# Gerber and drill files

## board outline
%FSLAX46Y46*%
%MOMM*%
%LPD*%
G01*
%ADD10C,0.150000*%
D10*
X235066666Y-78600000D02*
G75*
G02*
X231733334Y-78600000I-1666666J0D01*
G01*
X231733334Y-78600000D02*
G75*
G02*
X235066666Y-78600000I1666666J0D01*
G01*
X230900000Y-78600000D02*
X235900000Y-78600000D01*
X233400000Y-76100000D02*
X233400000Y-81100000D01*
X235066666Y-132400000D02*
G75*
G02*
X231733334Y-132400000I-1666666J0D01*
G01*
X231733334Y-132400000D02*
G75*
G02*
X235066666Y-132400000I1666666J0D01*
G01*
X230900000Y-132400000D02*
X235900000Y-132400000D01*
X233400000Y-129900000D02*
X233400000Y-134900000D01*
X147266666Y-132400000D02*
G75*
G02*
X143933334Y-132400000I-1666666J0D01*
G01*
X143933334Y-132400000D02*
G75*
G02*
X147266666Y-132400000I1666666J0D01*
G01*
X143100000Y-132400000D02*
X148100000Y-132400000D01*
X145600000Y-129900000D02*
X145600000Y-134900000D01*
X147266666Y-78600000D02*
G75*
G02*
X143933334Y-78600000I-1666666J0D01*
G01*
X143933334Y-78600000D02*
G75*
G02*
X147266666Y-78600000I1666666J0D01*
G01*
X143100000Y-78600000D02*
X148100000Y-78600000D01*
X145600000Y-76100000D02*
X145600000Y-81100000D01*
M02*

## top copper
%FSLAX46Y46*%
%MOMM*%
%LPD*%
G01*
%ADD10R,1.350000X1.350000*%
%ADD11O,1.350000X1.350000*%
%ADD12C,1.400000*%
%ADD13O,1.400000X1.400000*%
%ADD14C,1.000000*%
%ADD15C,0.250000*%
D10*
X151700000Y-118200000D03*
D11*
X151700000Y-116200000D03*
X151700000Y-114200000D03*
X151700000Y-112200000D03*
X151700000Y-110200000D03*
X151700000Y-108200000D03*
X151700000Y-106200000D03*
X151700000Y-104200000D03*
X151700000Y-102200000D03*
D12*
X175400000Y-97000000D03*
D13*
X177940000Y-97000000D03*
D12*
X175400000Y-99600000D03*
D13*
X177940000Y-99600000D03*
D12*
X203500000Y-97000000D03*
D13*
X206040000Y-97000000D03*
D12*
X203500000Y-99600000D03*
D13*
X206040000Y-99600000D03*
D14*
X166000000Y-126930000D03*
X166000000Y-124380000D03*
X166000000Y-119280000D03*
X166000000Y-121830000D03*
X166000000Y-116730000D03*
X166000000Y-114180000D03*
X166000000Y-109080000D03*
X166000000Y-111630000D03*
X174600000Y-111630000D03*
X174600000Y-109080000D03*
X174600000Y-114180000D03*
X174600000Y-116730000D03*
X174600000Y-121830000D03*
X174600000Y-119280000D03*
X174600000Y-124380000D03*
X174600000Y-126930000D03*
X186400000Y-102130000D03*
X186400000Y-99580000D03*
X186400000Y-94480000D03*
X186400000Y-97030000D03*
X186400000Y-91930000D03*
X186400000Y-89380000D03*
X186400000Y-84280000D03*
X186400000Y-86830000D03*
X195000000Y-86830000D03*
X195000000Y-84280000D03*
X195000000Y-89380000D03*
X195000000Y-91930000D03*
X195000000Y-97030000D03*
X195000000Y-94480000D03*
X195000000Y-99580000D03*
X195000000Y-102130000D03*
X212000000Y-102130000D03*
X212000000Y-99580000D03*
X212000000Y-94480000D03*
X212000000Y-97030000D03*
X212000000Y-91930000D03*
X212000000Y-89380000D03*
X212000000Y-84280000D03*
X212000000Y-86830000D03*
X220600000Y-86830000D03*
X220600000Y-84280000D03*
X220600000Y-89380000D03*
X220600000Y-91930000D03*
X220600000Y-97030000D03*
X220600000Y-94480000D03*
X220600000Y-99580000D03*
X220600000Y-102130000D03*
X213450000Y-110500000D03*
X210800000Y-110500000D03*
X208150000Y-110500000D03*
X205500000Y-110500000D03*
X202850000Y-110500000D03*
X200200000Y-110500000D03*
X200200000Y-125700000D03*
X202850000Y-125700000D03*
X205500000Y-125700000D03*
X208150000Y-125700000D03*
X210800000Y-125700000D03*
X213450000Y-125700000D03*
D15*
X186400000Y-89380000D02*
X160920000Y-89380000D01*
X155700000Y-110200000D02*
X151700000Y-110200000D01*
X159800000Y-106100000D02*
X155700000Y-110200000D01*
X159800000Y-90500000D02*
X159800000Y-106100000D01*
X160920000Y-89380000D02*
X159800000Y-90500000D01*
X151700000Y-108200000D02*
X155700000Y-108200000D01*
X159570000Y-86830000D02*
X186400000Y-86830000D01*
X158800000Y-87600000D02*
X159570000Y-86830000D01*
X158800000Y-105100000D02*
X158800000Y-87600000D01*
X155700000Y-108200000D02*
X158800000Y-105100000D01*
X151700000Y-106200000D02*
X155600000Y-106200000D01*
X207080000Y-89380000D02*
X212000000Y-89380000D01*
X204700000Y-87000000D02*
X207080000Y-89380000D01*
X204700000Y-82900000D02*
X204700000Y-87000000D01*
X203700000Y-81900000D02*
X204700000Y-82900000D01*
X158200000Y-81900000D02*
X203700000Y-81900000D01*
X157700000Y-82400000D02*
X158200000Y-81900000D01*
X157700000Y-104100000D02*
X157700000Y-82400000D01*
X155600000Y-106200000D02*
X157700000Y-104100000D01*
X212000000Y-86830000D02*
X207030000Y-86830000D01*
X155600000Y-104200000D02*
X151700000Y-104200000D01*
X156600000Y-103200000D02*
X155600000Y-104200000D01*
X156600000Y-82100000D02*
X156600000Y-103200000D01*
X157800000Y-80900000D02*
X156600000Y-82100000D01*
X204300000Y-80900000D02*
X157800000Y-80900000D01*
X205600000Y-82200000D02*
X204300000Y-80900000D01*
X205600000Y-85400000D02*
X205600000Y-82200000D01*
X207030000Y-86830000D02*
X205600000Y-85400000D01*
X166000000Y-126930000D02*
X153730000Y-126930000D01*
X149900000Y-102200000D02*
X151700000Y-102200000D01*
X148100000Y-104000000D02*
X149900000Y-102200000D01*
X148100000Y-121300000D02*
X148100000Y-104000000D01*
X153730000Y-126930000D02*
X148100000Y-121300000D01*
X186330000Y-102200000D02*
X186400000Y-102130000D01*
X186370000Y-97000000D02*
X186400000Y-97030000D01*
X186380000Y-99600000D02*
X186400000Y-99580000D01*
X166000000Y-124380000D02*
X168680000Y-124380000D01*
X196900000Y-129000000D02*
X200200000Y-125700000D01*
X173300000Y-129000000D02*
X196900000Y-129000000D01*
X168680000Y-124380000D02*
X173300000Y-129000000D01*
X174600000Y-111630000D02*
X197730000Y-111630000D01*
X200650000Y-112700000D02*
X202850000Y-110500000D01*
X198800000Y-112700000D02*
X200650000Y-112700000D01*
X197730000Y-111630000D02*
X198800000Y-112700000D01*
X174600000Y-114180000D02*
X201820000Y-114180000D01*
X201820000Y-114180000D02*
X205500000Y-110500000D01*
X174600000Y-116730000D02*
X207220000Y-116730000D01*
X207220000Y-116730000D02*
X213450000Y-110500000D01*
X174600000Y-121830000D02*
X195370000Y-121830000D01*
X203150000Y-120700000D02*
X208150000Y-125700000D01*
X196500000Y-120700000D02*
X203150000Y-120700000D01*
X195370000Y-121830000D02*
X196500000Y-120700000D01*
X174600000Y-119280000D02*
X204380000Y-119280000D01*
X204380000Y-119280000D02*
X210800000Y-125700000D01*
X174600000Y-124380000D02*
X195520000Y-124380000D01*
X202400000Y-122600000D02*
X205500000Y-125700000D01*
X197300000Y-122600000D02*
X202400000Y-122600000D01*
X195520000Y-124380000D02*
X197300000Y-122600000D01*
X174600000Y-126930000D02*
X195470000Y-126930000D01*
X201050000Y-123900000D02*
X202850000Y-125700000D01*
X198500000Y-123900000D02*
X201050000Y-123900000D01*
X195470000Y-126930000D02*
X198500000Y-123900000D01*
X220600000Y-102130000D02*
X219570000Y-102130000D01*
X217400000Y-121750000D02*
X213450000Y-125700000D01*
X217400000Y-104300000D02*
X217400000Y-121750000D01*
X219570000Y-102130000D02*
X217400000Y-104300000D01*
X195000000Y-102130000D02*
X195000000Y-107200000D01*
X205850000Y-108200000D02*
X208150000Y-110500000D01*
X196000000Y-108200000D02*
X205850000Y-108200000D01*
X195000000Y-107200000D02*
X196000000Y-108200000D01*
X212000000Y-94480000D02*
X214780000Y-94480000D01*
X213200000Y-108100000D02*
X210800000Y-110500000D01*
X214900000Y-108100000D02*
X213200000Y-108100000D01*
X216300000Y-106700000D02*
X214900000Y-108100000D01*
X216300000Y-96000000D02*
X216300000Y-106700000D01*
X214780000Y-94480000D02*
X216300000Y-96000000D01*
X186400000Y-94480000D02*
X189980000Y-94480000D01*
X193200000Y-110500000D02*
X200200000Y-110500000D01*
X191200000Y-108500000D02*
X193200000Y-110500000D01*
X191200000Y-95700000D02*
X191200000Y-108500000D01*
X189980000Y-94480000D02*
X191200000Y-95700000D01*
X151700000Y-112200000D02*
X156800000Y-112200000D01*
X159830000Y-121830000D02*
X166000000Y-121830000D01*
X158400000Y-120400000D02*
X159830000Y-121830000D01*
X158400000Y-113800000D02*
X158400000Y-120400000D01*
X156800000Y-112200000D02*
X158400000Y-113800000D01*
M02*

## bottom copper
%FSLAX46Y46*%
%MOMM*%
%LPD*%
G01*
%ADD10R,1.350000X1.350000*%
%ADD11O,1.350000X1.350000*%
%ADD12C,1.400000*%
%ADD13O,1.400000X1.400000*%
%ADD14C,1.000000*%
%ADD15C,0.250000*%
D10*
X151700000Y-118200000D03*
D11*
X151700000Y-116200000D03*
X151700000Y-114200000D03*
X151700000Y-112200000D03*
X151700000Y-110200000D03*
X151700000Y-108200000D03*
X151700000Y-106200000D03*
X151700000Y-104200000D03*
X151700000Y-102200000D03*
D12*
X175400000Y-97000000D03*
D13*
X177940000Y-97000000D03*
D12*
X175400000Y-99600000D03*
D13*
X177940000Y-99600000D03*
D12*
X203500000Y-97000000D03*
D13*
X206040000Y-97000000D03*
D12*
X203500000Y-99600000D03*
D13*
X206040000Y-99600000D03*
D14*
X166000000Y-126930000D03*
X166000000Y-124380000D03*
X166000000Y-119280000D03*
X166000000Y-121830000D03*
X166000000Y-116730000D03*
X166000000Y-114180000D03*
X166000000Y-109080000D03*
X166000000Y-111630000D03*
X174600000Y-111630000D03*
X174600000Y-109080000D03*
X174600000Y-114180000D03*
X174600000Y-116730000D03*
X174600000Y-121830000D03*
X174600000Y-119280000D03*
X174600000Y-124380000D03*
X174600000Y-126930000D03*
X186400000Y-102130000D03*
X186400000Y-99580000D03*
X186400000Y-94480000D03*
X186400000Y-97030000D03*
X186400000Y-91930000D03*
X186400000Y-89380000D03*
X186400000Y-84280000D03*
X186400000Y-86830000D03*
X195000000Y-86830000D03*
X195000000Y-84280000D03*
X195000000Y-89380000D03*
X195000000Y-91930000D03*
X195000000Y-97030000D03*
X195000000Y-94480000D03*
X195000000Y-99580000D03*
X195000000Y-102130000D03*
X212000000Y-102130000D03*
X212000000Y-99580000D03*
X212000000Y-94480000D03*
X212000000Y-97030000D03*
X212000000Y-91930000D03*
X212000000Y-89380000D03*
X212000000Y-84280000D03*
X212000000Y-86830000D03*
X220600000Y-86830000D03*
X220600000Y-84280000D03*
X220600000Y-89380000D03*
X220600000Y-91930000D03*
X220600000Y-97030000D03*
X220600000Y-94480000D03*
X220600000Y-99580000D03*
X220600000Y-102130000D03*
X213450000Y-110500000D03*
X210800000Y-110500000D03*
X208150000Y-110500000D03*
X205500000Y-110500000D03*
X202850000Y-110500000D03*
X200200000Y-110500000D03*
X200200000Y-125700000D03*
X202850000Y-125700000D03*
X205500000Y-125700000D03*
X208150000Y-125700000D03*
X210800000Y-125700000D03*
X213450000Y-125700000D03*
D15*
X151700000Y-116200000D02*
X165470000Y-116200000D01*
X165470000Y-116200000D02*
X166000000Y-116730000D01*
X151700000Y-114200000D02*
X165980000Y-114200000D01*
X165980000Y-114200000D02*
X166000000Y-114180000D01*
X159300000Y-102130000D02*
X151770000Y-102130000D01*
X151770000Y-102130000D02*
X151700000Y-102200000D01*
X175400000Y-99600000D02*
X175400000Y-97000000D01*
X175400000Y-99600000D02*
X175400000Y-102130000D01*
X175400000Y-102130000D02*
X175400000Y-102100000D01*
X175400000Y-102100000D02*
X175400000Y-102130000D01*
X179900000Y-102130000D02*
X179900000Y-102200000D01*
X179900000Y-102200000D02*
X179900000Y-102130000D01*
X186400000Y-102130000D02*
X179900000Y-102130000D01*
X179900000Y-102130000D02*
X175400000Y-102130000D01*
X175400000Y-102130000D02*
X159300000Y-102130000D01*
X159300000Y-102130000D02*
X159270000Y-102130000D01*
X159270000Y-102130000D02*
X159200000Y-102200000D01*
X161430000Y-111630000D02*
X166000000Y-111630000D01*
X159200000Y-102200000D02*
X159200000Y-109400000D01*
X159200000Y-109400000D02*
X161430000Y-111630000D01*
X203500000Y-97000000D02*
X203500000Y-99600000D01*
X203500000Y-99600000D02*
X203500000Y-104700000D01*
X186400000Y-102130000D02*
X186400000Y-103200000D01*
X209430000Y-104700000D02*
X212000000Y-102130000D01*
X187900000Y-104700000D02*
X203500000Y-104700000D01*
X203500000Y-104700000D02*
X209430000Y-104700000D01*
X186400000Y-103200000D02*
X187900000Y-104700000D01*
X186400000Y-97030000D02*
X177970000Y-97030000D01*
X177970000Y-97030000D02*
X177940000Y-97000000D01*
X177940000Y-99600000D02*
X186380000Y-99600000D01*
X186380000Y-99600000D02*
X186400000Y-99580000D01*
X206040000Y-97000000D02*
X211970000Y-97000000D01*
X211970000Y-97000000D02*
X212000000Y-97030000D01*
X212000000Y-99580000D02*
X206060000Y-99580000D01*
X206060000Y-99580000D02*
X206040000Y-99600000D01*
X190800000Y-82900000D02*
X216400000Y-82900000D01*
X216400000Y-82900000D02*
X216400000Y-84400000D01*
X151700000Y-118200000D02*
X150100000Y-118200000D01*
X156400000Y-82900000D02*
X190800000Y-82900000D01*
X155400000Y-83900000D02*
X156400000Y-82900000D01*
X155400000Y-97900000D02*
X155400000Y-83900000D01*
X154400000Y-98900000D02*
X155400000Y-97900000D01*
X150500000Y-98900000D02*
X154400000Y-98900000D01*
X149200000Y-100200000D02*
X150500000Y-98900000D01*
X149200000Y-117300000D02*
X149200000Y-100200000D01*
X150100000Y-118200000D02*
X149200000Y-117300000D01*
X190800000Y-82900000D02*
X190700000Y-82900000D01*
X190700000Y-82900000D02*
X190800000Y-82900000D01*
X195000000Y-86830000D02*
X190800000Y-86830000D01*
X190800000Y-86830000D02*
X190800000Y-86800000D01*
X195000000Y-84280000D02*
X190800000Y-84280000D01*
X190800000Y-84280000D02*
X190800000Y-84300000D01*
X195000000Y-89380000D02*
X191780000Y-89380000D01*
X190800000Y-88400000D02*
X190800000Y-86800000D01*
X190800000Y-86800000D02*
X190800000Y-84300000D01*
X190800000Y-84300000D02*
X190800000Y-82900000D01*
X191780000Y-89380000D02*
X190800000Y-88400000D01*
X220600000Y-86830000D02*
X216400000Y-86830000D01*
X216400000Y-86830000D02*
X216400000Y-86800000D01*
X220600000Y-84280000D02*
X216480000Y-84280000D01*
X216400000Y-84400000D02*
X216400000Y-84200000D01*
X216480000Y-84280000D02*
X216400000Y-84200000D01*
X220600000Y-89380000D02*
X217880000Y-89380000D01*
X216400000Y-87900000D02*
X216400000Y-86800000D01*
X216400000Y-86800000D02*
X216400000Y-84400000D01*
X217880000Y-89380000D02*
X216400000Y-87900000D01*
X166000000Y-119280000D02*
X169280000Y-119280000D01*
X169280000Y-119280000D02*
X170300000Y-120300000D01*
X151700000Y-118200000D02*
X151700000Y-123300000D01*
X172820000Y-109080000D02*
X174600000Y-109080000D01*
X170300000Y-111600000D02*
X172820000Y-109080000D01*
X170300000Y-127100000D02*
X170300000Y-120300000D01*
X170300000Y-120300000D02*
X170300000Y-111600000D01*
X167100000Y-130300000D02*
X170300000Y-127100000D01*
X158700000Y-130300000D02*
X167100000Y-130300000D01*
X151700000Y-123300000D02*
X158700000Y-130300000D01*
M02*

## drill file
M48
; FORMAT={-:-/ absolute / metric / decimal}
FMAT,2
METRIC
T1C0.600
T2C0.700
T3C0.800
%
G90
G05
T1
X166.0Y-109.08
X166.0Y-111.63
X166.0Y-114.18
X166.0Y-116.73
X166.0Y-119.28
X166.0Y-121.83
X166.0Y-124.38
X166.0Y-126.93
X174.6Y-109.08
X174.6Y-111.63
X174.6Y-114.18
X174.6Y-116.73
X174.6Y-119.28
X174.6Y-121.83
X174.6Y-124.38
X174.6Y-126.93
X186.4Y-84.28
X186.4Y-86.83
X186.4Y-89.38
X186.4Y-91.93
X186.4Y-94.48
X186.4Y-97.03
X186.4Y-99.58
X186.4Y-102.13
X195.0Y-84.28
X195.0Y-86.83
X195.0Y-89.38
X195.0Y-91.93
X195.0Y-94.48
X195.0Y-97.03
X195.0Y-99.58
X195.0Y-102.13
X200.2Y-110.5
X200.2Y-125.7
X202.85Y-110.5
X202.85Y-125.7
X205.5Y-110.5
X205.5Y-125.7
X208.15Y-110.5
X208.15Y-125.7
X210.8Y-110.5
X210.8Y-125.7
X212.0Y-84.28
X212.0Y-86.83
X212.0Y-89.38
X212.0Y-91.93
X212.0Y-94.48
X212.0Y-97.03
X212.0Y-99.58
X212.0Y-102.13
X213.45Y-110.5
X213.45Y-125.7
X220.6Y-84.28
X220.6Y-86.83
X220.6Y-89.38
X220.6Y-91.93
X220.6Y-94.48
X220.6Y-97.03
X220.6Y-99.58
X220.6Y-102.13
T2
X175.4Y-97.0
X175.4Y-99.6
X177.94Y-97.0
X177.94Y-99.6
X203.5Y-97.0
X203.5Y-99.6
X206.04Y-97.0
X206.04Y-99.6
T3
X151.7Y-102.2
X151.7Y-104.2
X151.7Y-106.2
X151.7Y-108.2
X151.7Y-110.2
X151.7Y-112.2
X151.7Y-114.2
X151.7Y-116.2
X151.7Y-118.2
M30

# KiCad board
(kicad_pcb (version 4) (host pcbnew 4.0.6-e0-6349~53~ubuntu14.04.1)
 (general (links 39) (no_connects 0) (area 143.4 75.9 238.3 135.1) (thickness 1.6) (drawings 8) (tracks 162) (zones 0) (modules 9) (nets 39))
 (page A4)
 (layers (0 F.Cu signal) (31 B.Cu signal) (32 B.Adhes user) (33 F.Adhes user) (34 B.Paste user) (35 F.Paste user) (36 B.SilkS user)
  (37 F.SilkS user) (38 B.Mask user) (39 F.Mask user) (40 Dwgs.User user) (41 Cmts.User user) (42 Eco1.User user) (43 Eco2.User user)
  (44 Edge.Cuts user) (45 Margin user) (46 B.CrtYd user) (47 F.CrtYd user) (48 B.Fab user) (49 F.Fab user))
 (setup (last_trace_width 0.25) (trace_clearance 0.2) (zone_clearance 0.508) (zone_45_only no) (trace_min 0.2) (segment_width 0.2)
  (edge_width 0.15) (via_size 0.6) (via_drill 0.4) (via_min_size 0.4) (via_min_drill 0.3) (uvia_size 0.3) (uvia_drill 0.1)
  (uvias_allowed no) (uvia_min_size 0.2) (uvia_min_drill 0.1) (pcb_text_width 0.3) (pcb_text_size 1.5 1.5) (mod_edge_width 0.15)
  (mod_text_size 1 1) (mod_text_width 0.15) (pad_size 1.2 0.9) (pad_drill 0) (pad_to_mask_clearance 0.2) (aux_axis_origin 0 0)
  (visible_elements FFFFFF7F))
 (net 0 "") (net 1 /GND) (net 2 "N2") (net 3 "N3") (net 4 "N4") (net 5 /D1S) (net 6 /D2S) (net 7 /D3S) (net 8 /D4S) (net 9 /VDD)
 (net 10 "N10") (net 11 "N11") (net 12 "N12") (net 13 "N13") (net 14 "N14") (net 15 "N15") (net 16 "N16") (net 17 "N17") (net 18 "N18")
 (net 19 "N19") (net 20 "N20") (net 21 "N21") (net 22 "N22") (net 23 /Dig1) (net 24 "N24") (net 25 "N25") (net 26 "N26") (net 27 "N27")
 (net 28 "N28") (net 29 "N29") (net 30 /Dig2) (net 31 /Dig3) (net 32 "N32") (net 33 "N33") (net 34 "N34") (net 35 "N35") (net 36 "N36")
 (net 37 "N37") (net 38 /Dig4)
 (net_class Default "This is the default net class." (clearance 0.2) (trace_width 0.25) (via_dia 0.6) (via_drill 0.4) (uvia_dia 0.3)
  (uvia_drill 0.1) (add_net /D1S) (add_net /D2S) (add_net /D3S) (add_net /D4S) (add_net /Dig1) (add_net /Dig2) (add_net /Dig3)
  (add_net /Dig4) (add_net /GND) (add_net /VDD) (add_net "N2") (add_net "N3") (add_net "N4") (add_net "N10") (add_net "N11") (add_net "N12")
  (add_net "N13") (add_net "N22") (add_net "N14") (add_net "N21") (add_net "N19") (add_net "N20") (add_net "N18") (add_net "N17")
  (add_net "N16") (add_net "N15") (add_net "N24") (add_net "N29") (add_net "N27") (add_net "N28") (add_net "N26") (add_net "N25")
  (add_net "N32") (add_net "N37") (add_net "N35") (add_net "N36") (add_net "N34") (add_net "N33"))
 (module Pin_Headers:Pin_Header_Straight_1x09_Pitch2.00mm (layer F.Cu) (at 151.7 118.2 180)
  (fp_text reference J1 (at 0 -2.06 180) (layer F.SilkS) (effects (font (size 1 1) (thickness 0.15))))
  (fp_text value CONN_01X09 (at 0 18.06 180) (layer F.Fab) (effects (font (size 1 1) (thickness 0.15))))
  (pad 1 thru_hole rect (at 0 0 180) (size 1.35 1.35) (drill 0.8) (layers *.Cu *.Mask) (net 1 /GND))
  (pad 2 thru_hole oval (at 0 2 180) (size 1.35 1.35) (drill 0.8) (layers *.Cu *.Mask) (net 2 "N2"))
  (pad 3 thru_hole oval (at 0 4 180) (size 1.35 1.35) (drill 0.8) (layers *.Cu *.Mask) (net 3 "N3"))
  (pad 4 thru_hole oval (at 0 6 180) (size 1.35 1.35) (drill 0.8) (layers *.Cu *.Mask) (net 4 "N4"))
  (pad 5 thru_hole oval (at 0 8 180) (size 1.35 1.35) (drill 0.8) (layers *.Cu *.Mask) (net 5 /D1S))
  (pad 6 thru_hole oval (at 0 10 180) (size 1.35 1.35) (drill 0.8) (layers *.Cu *.Mask) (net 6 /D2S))
  (pad 7 thru_hole oval (at 0 12 180) (size 1.35 1.35) (drill 0.8) (layers *.Cu *.Mask) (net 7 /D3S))
  (pad 8 thru_hole oval (at 0 14 180) (size 1.35 1.35) (drill 0.8) (layers *.Cu *.Mask) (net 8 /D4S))
  (pad 9 thru_hole oval (at 0 16 180) (size 1.35 1.35) (drill 0.8) (layers *.Cu *.Mask) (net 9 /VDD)))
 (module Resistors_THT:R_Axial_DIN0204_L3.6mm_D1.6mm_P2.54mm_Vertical (layer F.Cu) (at 175.4 97)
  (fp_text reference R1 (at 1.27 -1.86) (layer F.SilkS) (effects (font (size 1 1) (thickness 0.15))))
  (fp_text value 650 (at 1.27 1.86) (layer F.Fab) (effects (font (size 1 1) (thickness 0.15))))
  (pad 1 thru_hole circle (at 0 0) (size 1.4 1.4) (drill 0.7) (layers *.Cu *.Mask) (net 9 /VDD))
  (pad 2 thru_hole oval (at 2.54 0) (size 1.4 1.4) (drill 0.7) (layers *.Cu *.Mask) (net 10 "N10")))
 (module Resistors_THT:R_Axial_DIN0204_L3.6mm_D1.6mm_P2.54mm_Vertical (layer F.Cu) (at 175.4 99.6)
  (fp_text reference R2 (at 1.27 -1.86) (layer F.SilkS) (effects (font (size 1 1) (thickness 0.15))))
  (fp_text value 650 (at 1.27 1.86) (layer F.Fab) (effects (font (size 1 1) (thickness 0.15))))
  (pad 1 thru_hole circle (at 0 0) (size 1.4 1.4) (drill 0.7) (layers *.Cu *.Mask) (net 9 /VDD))
  (pad 2 thru_hole oval (at 2.54 0) (size 1.4 1.4) (drill 0.7) (layers *.Cu *.Mask) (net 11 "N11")))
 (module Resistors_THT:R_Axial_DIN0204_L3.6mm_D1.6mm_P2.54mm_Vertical (layer F.Cu) (at 203.5 97)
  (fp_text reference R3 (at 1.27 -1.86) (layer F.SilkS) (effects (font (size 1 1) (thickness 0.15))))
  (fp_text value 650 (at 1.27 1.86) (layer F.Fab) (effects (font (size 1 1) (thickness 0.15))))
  (pad 1 thru_hole circle (at 0 0) (size 1.4 1.4) (drill 0.7) (layers *.Cu *.Mask) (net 9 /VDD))
  (pad 2 thru_hole oval (at 2.54 0) (size 1.4 1.4) (drill 0.7) (layers *.Cu *.Mask) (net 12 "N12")))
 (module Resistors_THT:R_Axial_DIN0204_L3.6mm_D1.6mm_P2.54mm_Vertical (layer F.Cu) (at 203.5 99.6)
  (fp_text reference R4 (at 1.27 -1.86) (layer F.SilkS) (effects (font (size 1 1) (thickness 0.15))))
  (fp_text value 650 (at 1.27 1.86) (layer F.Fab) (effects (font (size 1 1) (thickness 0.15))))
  (pad 1 thru_hole circle (at 0 0) (size 1.4 1.4) (drill 0.7) (layers *.Cu *.Mask) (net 9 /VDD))
  (pad 2 thru_hole oval (at 2.54 0) (size 1.4 1.4) (drill 0.7) (layers *.Cu *.Mask) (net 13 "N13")))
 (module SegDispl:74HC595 (layer F.Cu) (at 174.6 127.7 180)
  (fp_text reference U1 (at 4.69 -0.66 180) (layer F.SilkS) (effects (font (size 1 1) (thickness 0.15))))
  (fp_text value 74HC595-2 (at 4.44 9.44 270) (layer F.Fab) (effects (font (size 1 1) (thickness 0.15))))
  (pad 16 thru_hole circle (at 8.6 0.77 180) (size 1 1) (drill 0.6) (layers *.Cu *.Mask) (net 9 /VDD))
  (pad 15 thru_hole circle (at 8.6 3.32 180) (size 1 1) (drill 0.6) (layers *.Cu *.Mask) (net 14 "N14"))
  (pad 13 thru_hole circle (at 8.6 8.42 180) (size 1 1) (drill 0.6) (layers *.Cu *.Mask) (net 1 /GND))
  (pad 14 thru_hole circle (at 8.6 5.87 180) (size 1 1) (drill 0.6) (layers *.Cu *.Mask) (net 4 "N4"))
  (pad 12 thru_hole circle (at 8.6 10.97 180) (size 1 1) (drill 0.6) (layers *.Cu *.Mask) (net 2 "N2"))
  (pad 11 thru_hole circle (at 8.6 13.52 180) (size 1 1) (drill 0.6) (layers *.Cu *.Mask) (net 3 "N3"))
  (pad 9 thru_hole circle (at 8.6 18.62 180) (size 1 1) (drill 0.6) (layers *.Cu *.Mask) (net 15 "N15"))
  (pad 10 thru_hole circle (at 8.6 16.07 180) (size 1 1) (drill 0.6) (layers *.Cu *.Mask) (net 9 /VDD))
  (pad 7 thru_hole circle (at 0 16.07 180) (size 1 1) (drill 0.6) (layers *.Cu *.Mask) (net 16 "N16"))
  (pad 8 thru_hole circle (at 0 18.62 180) (size 1 1) (drill 0.6) (layers *.Cu *.Mask) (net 1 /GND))
  (pad 6 thru_hole circle (at 0 13.52 180) (size 1 1) (drill 0.6) (layers *.Cu *.Mask) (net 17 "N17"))
  (pad 5 thru_hole circle (at 0 10.97 180) (size 1 1) (drill 0.6) (layers *.Cu *.Mask) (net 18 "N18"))
  (pad 3 thru_hole circle (at 0 5.87 180) (size 1 1) (drill 0.6) (layers *.Cu *.Mask) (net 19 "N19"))
  (pad 4 thru_hole circle (at 0 8.42 180) (size 1 1) (drill 0.6) (layers *.Cu *.Mask) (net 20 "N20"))
  (pad 2 thru_hole circle (at 0 3.32 180) (size 1 1) (drill 0.6) (layers *.Cu *.Mask) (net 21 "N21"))
  (pad 1 thru_hole circle (at 0 0.77 180) (size 1 1) (drill 0.6) (layers *.Cu *.Mask) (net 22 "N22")))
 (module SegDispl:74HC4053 (layer F.Cu) (at 195 102.9 180)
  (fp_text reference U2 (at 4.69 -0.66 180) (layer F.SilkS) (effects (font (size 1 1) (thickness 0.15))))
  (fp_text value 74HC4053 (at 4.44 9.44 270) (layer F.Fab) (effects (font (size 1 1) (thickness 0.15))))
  (pad 16 thru_hole circle (at 8.6 0.77 180) (size 1 1) (drill 0.6) (layers *.Cu *.Mask) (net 9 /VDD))
  (pad 15 thru_hole circle (at 8.6 3.32 180) (size 1 1) (drill 0.6) (layers *.Cu *.Mask) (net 11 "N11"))
  (pad 13 thru_hole circle (at 8.6 8.42 180) (size 1 1) (drill 0.6) (layers *.Cu *.Mask) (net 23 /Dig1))
  (pad 14 thru_hole circle (at 8.6 5.87 180) (size 1 1) (drill 0.6) (layers *.Cu *.Mask) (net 10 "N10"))
  (pad 12 thru_hole circle (at 8.6 10.97 180) (size 1 1) (drill 0.6) (layers *.Cu *.Mask) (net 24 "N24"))
  (pad 11 thru_hole circle (at 8.6 13.52 180) (size 1 1) (drill 0.6) (layers *.Cu *.Mask) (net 5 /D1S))
  (pad 9 thru_hole circle (at 8.6 18.62 180) (size 1 1) (drill 0.6) (layers *.Cu *.Mask) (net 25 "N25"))
  (pad 10 thru_hole circle (at 8.6 16.07 180) (size 1 1) (drill 0.6) (layers *.Cu *.Mask) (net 6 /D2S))
  (pad 7 thru_hole circle (at 0 16.07 180) (size 1 1) (drill 0.6) (layers *.Cu *.Mask) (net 1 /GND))
  (pad 8 thru_hole circle (at 0 18.62 180) (size 1 1) (drill 0.6) (layers *.Cu *.Mask) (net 1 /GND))
  (pad 6 thru_hole circle (at 0 13.52 180) (size 1 1) (drill 0.6) (layers *.Cu *.Mask) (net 1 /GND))
  (pad 5 thru_hole circle (at 0 10.97 180) (size 1 1) (drill 0.6) (layers *.Cu *.Mask) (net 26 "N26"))
  (pad 3 thru_hole circle (at 0 5.87 180) (size 1 1) (drill 0.6) (layers *.Cu *.Mask) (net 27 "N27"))
  (pad 4 thru_hole circle (at 0 8.42 180) (size 1 1) (drill 0.6) (layers *.Cu *.Mask) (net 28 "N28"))
  (pad 2 thru_hole circle (at 0 3.32 180) (size 1 1) (drill 0.6) (layers *.Cu *.Mask) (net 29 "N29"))
  (pad 1 thru_hole circle (at 0 0.77 180) (size 1 1) (drill 0.6) (layers *.Cu *.Mask) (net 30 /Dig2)))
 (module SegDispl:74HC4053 (layer F.Cu) (at 220.6 102.9 180)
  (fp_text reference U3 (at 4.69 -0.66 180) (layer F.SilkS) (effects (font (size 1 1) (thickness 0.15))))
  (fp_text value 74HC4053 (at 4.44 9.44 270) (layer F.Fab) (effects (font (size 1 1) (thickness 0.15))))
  (pad 16 thru_hole circle (at 8.6 0.77 180) (size 1 1) (drill 0.6) (layers *.Cu *.Mask) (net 9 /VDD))
  (pad 15 thru_hole circle (at 8.6 3.32 180) (size 1 1) (drill 0.6) (layers *.Cu *.Mask) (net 13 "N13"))
  (pad 13 thru_hole circle (at 8.6 8.42 180) (size 1 1) (drill 0.6) (layers *.Cu *.Mask) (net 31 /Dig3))
  (pad 14 thru_hole circle (at 8.6 5.87 180) (size 1 1) (drill 0.6) (layers *.Cu *.Mask) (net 12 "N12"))
  (pad 12 thru_hole circle (at 8.6 10.97 180) (size 1 1) (drill 0.6) (layers *.Cu *.Mask) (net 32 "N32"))
  (pad 11 thru_hole circle (at 8.6 13.52 180) (size 1 1) (drill 0.6) (layers *.Cu *.Mask) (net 7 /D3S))
  (pad 9 thru_hole circle (at 8.6 18.62 180) (size 1 1) (drill 0.6) (layers *.Cu *.Mask) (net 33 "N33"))
  (pad 10 thru_hole circle (at 8.6 16.07 180) (size 1 1) (drill 0.6) (layers *.Cu *.Mask) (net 8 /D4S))
  (pad 7 thru_hole circle (at 0 16.07 180) (size 1 1) (drill 0.6) (layers *.Cu *.Mask) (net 1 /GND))
  (pad 8 thru_hole circle (at 0 18.62 180) (size 1 1) (drill 0.6) (layers *.Cu *.Mask) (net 1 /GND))
  (pad 6 thru_hole circle (at 0 13.52 180) (size 1 1) (drill 0.6) (layers *.Cu *.Mask) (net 1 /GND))
  (pad 5 thru_hole circle (at 0 10.97 180) (size 1 1) (drill 0.6) (layers *.Cu *.Mask) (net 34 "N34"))
  (pad 3 thru_hole circle (at 0 5.87 180) (size 1 1) (drill 0.6) (layers *.Cu *.Mask) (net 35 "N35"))
  (pad 4 thru_hole circle (at 0 8.42 180) (size 1 1) (drill 0.6) (layers *.Cu *.Mask) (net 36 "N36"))
  (pad 2 thru_hole circle (at 0 3.32 180) (size 1 1) (drill 0.6) (layers *.Cu *.Mask) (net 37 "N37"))
  (pad 1 thru_hole circle (at 0 0.77 180) (size 1 1) (drill 0.6) (layers *.Cu *.Mask) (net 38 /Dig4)))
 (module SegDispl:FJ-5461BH (layer F.Cu) (at 181.4 108.5)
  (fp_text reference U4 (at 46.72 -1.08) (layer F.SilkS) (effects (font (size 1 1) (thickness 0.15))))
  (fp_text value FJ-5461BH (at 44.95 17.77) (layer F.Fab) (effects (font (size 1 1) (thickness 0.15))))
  (pad 7 thru_hole circle (at 32.05 2) (size 1 1) (drill 0.6) (layers *.Cu *.Mask) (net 18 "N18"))
  (pad 8 thru_hole circle (at 29.4 2) (size 1 1) (drill 0.6) (layers *.Cu *.Mask) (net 31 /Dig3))
  (pad 9 thru_hole circle (at 26.75 2) (size 1 1) (drill 0.6) (layers *.Cu *.Mask) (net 30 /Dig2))
  (pad 10 thru_hole circle (at 24.1 2) (size 1 1) (drill 0.6) (layers *.Cu *.Mask) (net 17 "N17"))
  (pad 11 thru_hole circle (at 21.45 2) (size 1 1) (drill 0.6) (layers *.Cu *.Mask) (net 16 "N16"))
  (pad 12 thru_hole circle (at 18.8 2) (size 1 1) (drill 0.6) (layers *.Cu *.Mask) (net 23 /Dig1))
  (pad 1 thru_hole circle (at 18.8 17.2) (size 1 1) (drill 0.6) (layers *.Cu *.Mask) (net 14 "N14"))
  (pad 2 thru_hole circle (at 21.45 17.2) (size 1 1) (drill 0.6) (layers *.Cu *.Mask) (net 22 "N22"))
  (pad 3 thru_hole circle (at 24.1 17.2) (size 1 1) (drill 0.6) (layers *.Cu *.Mask) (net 21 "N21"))
  (pad 4 thru_hole circle (at 26.75 17.2) (size 1 1) (drill 0.6) (layers *.Cu *.Mask) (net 19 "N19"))
  (pad 5 thru_hole circle (at 29.4 17.2) (size 1 1) (drill 0.6) (layers *.Cu *.Mask) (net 20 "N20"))
  (pad 6 thru_hole circle (at 32.05 17.2) (size 1 1) (drill 0.6) (layers *.Cu *.Mask) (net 38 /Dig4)))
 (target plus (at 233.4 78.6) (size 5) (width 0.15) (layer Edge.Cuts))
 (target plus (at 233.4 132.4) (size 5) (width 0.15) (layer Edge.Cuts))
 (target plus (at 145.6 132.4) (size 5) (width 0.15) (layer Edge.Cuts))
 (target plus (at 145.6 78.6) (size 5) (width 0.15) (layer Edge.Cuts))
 (segment (start 151.7 116.2) (end 165.47 116.2) (width 0.25) (layer B.Cu) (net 2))
 (segment (start 165.47 116.2) (end 166 116.73) (width 0.25) (layer B.Cu) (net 2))
 (segment (start 151.7 114.2) (end 165.98 114.2) (width 0.25) (layer B.Cu) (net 3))
 (segment (start 165.98 114.2) (end 166 114.18) (width 0.25) (layer B.Cu) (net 3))
 (segment (start 186.4 89.38) (end 160.92 89.38) (width 0.25) (layer F.Cu) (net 5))
 (segment (start 155.7 110.2) (end 151.7 110.2) (width 0.25) (layer F.Cu) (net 5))
 (segment (start 159.8 106.1) (end 155.7 110.2) (width 0.25) (layer F.Cu) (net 5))
 (segment (start 159.8 90.5) (end 159.8 106.1) (width 0.25) (layer F.Cu) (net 5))
 (segment (start 160.92 89.38) (end 159.8 90.5) (width 0.25) (layer F.Cu) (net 5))
 (segment (start 151.7 108.2) (end 155.7 108.2) (width 0.25) (layer F.Cu) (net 6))
 (segment (start 159.57 86.83) (end 186.4 86.83) (width 0.25) (layer F.Cu) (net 6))
 (segment (start 158.8 87.6) (end 159.57 86.83) (width 0.25) (layer F.Cu) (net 6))
 (segment (start 158.8 105.1) (end 158.8 87.6) (width 0.25) (layer F.Cu) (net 6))
 (segment (start 155.7 108.2) (end 158.8 105.1) (width 0.25) (layer F.Cu) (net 6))
 (segment (start 151.7 106.2) (end 155.6 106.2) (width 0.25) (layer F.Cu) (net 7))
 (segment (start 207.08 89.38) (end 212 89.38) (width 0.25) (layer F.Cu) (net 7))
 (segment (start 204.7 87) (end 207.08 89.38) (width 0.25) (layer F.Cu) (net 7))
 (segment (start 204.7 82.9) (end 204.7 87) (width 0.25) (layer F.Cu) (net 7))
 (segment (start 203.7 81.9) (end 204.7 82.9) (width 0.25) (layer F.Cu) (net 7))
 (segment (start 158.2 81.9) (end 203.7 81.9) (width 0.25) (layer F.Cu) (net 7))
 (segment (start 157.7 82.4) (end 158.2 81.9) (width 0.25) (layer F.Cu) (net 7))
 (segment (start 157.7 104.1) (end 157.7 82.4) (width 0.25) (layer F.Cu) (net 7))
 (segment (start 155.6 106.2) (end 157.7 104.1) (width 0.25) (layer F.Cu) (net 7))
 (segment (start 212 86.83) (end 207.03 86.83) (width 0.25) (layer F.Cu) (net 8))
 (segment (start 155.6 104.2) (end 151.7 104.2) (width 0.25) (layer F.Cu) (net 8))
 (segment (start 156.6 103.2) (end 155.6 104.2) (width 0.25) (layer F.Cu) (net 8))
 (segment (start 156.6 82.1) (end 156.6 103.2) (width 0.25) (layer F.Cu) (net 8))
 (segment (start 157.8 80.9) (end 156.6 82.1) (width 0.25) (layer F.Cu) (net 8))
 (segment (start 204.3 80.9) (end 157.8 80.9) (width 0.25) (layer F.Cu) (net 8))
 (segment (start 205.6 82.2) (end 204.3 80.9) (width 0.25) (layer F.Cu) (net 8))
 (segment (start 205.6 85.4) (end 205.6 82.2) (width 0.25) (layer F.Cu) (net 8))
 (segment (start 207.03 86.83) (end 205.6 85.4) (width 0.25) (layer F.Cu) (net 8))
 (segment (start 159.3 102.13) (end 151.77 102.13) (width 0.25) (layer B.Cu) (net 9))
 (segment (start 151.77 102.13) (end 151.7 102.2) (width 0.25) (layer B.Cu) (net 9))
 (segment (start 166 126.93) (end 153.73 126.93) (width 0.25) (layer F.Cu) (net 9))
 (segment (start 149.9 102.2) (end 151.7 102.2) (width 0.25) (layer F.Cu) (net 9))
 (segment (start 148.1 104) (end 149.9 102.2) (width 0.25) (layer F.Cu) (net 9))
 (segment (start 148.1 121.3) (end 148.1 104) (width 0.25) (layer F.Cu) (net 9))
 (segment (start 153.73 126.93) (end 148.1 121.3) (width 0.25) (layer F.Cu) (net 9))
 (segment (start 175.4 99.6) (end 175.4 97) (width 0.25) (layer B.Cu) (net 9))
 (segment (start 175.4 99.6) (end 175.4 102.13) (width 0.25) (layer B.Cu) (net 9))
 (segment (start 175.4 102.13) (end 175.4 102.1) (width 0.25) (layer B.Cu) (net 9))
 (segment (start 175.4 102.1) (end 175.4 102.13) (width 0.25) (layer B.Cu) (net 9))
 (segment (start 179.9 102.13) (end 179.9 102.2) (width 0.25) (layer B.Cu) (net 9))
 (segment (start 179.9 102.2) (end 179.9 102.13) (width 0.25) (layer B.Cu) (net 9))
 (segment (start 186.4 102.13) (end 179.9 102.13) (width 0.25) (layer B.Cu) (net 9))
 (segment (start 179.9 102.13) (end 175.4 102.13) (width 0.25) (layer B.Cu) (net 9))
 (segment (start 175.4 102.13) (end 159.3 102.13) (width 0.25) (layer B.Cu) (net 9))
 (segment (start 159.3 102.13) (end 159.27 102.13) (width 0.25) (layer B.Cu) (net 9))
 (segment (start 159.27 102.13) (end 159.2 102.2) (width 0.25) (layer B.Cu) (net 9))
 (segment (start 161.43 111.63) (end 166 111.63) (width 0.25) (layer B.Cu) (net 9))
 (segment (start 159.2 102.2) (end 159.2 109.4) (width 0.25) (layer B.Cu) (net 9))
 (segment (start 159.2 109.4) (end 161.43 111.63) (width 0.25) (layer B.Cu) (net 9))
 (segment (start 203.5 97) (end 203.5 99.6) (width 0.25) (layer B.Cu) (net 9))
 (segment (start 203.5 99.6) (end 203.5 104.7) (width 0.25) (layer B.Cu) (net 9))
 (segment (start 186.4 102.13) (end 186.4 103.2) (width 0.25) (layer B.Cu) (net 9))
 (segment (start 209.43 104.7) (end 212 102.13) (width 0.25) (layer B.Cu) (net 9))
 (segment (start 187.9 104.7) (end 203.5 104.7) (width 0.25) (layer B.Cu) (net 9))
 (segment (start 203.5 104.7) (end 209.43 104.7) (width 0.25) (layer B.Cu) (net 9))
 (segment (start 186.4 103.2) (end 187.9 104.7) (width 0.25) (layer B.Cu) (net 9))
 (segment (start 186.33 102.2) (end 186.4 102.13) (width 0.25) (layer F.Cu) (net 9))
 (segment (start 186.4 97.03) (end 177.97 97.03) (width 0.25) (layer B.Cu) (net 10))
 (segment (start 177.97 97.03) (end 177.94 97) (width 0.25) (layer B.Cu) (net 10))
 (segment (start 186.37 97) (end 186.4 97.03) (width 0.25) (layer F.Cu) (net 10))
 (segment (start 177.94 99.6) (end 186.38 99.6) (width 0.25) (layer B.Cu) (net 11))
 (segment (start 186.38 99.6) (end 186.4 99.58) (width 0.25) (layer B.Cu) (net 11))
 (segment (start 186.38 99.6) (end 186.4 99.58) (width 0.25) (layer F.Cu) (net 11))
 (segment (start 206.04 97) (end 211.97 97) (width 0.25) (layer B.Cu) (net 12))
 (segment (start 211.97 97) (end 212 97.03) (width 0.25) (layer B.Cu) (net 12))
 (segment (start 212 99.58) (end 206.06 99.58) (width 0.25) (layer B.Cu) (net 13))
 (segment (start 206.06 99.58) (end 206.04 99.6) (width 0.25) (layer B.Cu) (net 13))
 (segment (start 166 124.38) (end 168.68 124.38) (width 0.25) (layer F.Cu) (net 14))
 (segment (start 196.9 129) (end 200.2 125.7) (width 0.25) (layer F.Cu) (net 14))
 (segment (start 173.3 129) (end 196.9 129) (width 0.25) (layer F.Cu) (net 14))
 (segment (start 168.68 124.38) (end 173.3 129) (width 0.25) (layer F.Cu) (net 14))
 (segment (start 190.8 82.9) (end 216.4 82.9) (width 0.25) (layer B.Cu) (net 1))
 (segment (start 216.4 82.9) (end 216.4 84.4) (width 0.25) (layer B.Cu) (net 1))
 (segment (start 151.7 118.2) (end 150.1 118.2) (width 0.25) (layer B.Cu) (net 1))
 (segment (start 156.4 82.9) (end 190.8 82.9) (width 0.25) (layer B.Cu) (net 1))
 (segment (start 155.4 83.9) (end 156.4 82.9) (width 0.25) (layer B.Cu) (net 1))
 (segment (start 155.4 97.9) (end 155.4 83.9) (width 0.25) (layer B.Cu) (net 1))
 (segment (start 154.4 98.9) (end 155.4 97.9) (width 0.25) (layer B.Cu) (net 1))
 (segment (start 150.5 98.9) (end 154.4 98.9) (width 0.25) (layer B.Cu) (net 1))
 (segment (start 149.2 100.2) (end 150.5 98.9) (width 0.25) (layer B.Cu) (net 1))
 (segment (start 149.2 117.3) (end 149.2 100.2) (width 0.25) (layer B.Cu) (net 1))
 (segment (start 150.1 118.2) (end 149.2 117.3) (width 0.25) (layer B.Cu) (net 1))
 (segment (start 190.8 82.9) (end 190.7 82.9) (width 0.25) (layer B.Cu) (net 1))
 (segment (start 190.7 82.9) (end 190.8 82.9) (width 0.25) (layer B.Cu) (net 1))
 (segment (start 195 86.83) (end 190.8 86.83) (width 0.25) (layer B.Cu) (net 1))
 (segment (start 190.8 86.83) (end 190.8 86.8) (width 0.25) (layer B.Cu) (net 1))
 (segment (start 195 84.28) (end 190.8 84.28) (width 0.25) (layer B.Cu) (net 1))
 (segment (start 190.8 84.28) (end 190.8 84.3) (width 0.25) (layer B.Cu) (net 1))
 (segment (start 195 89.38) (end 191.78 89.38) (width 0.25) (layer B.Cu) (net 1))
 (segment (start 190.8 88.4) (end 190.8 86.8) (width 0.25) (layer B.Cu) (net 1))
 (segment (start 190.8 86.8) (end 190.8 84.3) (width 0.25) (layer B.Cu) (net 1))
 (segment (start 190.8 84.3) (end 190.8 82.9) (width 0.25) (layer B.Cu) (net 1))
 (segment (start 191.78 89.38) (end 190.8 88.4) (width 0.25) (layer B.Cu) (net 1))
 (segment (start 220.6 86.83) (end 216.4 86.83) (width 0.25) (layer B.Cu) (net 1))
 (segment (start 216.4 86.83) (end 216.4 86.8) (width 0.25) (layer B.Cu) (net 1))
 (segment (start 220.6 84.28) (end 216.48 84.28) (width 0.25) (layer B.Cu) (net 1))
 (segment (start 216.4 84.4) (end 216.4 84.2) (width 0.25) (layer B.Cu) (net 1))
 (segment (start 216.48 84.28) (end 216.4 84.2) (width 0.25) (layer B.Cu) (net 1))
 (segment (start 220.6 89.38) (end 217.88 89.38) (width 0.25) (layer B.Cu) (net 1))
 (segment (start 216.4 87.9) (end 216.4 86.8) (width 0.25) (layer B.Cu) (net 1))
 (segment (start 216.4 86.8) (end 216.4 84.4) (width 0.25) (layer B.Cu) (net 1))
 (segment (start 217.88 89.38) (end 216.4 87.9) (width 0.25) (layer B.Cu) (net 1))
 (segment (start 166 119.28) (end 169.28 119.28) (width 0.25) (layer B.Cu) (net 1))
 (segment (start 169.28 119.28) (end 170.3 120.3) (width 0.25) (layer B.Cu) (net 1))
 (segment (start 151.7 118.2) (end 151.7 123.3) (width 0.25) (layer B.Cu) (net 1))
 (segment (start 172.82 109.08) (end 174.6 109.08) (width 0.25) (layer B.Cu) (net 1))
 (segment (start 170.3 111.6) (end 172.82 109.08) (width 0.25) (layer B.Cu) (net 1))
 (segment (start 170.3 127.1) (end 170.3 120.3) (width 0.25) (layer B.Cu) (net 1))
 (segment (start 170.3 120.3) (end 170.3 111.6) (width 0.25) (layer B.Cu) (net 1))
 (segment (start 167.1 130.3) (end 170.3 127.1) (width 0.25) (layer B.Cu) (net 1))
 (segment (start 158.7 130.3) (end 167.1 130.3) (width 0.25) (layer B.Cu) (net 1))
 (segment (start 151.7 123.3) (end 158.7 130.3) (width 0.25) (layer B.Cu) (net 1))
 (segment (start 174.6 111.63) (end 197.73 111.63) (width 0.25) (layer F.Cu) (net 16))
 (segment (start 200.65 112.7) (end 202.85 110.5) (width 0.25) (layer F.Cu) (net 16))
 (segment (start 198.8 112.7) (end 200.65 112.7) (width 0.25) (layer F.Cu) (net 16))
 (segment (start 197.73 111.63) (end 198.8 112.7) (width 0.25) (layer F.Cu) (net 16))
 (segment (start 174.6 114.18) (end 201.82 114.18) (width 0.25) (layer F.Cu) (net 17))
 (segment (start 201.82 114.18) (end 205.5 110.5) (width 0.25) (layer F.Cu) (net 17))
 (segment (start 174.6 116.73) (end 207.22 116.73) (width 0.25) (layer F.Cu) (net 18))
 (segment (start 207.22 116.73) (end 213.45 110.5) (width 0.25) (layer F.Cu) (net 18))
 (segment (start 174.6 121.83) (end 195.37 121.83) (width 0.25) (layer F.Cu) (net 19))
 (segment (start 203.15 120.7) (end 208.15 125.7) (width 0.25) (layer F.Cu) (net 19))
 (segment (start 196.5 120.7) (end 203.15 120.7) (width 0.25) (layer F.Cu) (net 19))
 (segment (start 195.37 121.83) (end 196.5 120.7) (width 0.25) (layer F.Cu) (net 19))
 (segment (start 174.6 119.28) (end 204.38 119.28) (width 0.25) (layer F.Cu) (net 20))
 (segment (start 204.38 119.28) (end 210.8 125.7) (width 0.25) (layer F.Cu) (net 20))
 (segment (start 174.6 124.38) (end 195.52 124.38) (width 0.25) (layer F.Cu) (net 21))
 (segment (start 202.4 122.6) (end 205.5 125.7) (width 0.25) (layer F.Cu) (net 21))
 (segment (start 197.3 122.6) (end 202.4 122.6) (width 0.25) (layer F.Cu) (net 21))
 (segment (start 195.52 124.38) (end 197.3 122.6) (width 0.25) (layer F.Cu) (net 21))
 (segment (start 174.6 126.93) (end 195.47 126.93) (width 0.25) (layer F.Cu) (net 22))
 (segment (start 201.05 123.9) (end 202.85 125.7) (width 0.25) (layer F.Cu) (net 22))
 (segment (start 198.5 123.9) (end 201.05 123.9) (width 0.25) (layer F.Cu) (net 22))
 (segment (start 195.47 126.93) (end 198.5 123.9) (width 0.25) (layer F.Cu) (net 22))
 (segment (start 220.6 102.13) (end 219.57 102.13) (width 0.25) (layer F.Cu) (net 38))
 (segment (start 217.4 121.75) (end 213.45 125.7) (width 0.25) (layer F.Cu) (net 38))
 (segment (start 217.4 104.3) (end 217.4 121.75) (width 0.25) (layer F.Cu) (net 38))
 (segment (start 219.57 102.13) (end 217.4 104.3) (width 0.25) (layer F.Cu) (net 38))
 (segment (start 195 102.13) (end 195 107.2) (width 0.25) (layer F.Cu) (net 30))
 (segment (start 205.85 108.2) (end 208.15 110.5) (width 0.25) (layer F.Cu) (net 30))
 (segment (start 196 108.2) (end 205.85 108.2) (width 0.25) (layer F.Cu) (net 30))
 (segment (start 195 107.2) (end 196 108.2) (width 0.25) (layer F.Cu) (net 30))
 (segment (start 212 94.48) (end 214.78 94.48) (width 0.25) (layer F.Cu) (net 31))
 (segment (start 213.2 108.1) (end 210.8 110.5) (width 0.25) (layer F.Cu) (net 31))
 (segment (start 214.9 108.1) (end 213.2 108.1) (width 0.25) (layer F.Cu) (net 31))
 (segment (start 216.3 106.7) (end 214.9 108.1) (width 0.25) (layer F.Cu) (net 31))
 (segment (start 216.3 96) (end 216.3 106.7) (width 0.25) (layer F.Cu) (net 31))
 (segment (start 214.78 94.48) (end 216.3 96) (width 0.25) (layer F.Cu) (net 31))
 (segment (start 186.4 94.48) (end 189.98 94.48) (width 0.25) (layer F.Cu) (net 23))
 (segment (start 193.2 110.5) (end 200.2 110.5) (width 0.25) (layer F.Cu) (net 23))
 (segment (start 191.2 108.5) (end 193.2 110.5) (width 0.25) (layer F.Cu) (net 23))
 (segment (start 191.2 95.7) (end 191.2 108.5) (width 0.25) (layer F.Cu) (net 23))
 (segment (start 189.98 94.48) (end 191.2 95.7) (width 0.25) (layer F.Cu) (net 23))
 (segment (start 151.7 112.2) (end 156.8 112.2) (width 0.25) (layer F.Cu) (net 4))
 (segment (start 159.83 121.83) (end 166 121.83) (width 0.25) (layer F.Cu) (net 4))
 (segment (start 158.4 120.4) (end 159.83 121.83) (width 0.25) (layer F.Cu) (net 4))
 (segment (start 158.4 113.8) (end 158.4 120.4) (width 0.25) (layer F.Cu) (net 4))
 (segment (start 156.8 112.2) (end 158.4 113.8) (width 0.25) (layer F.Cu) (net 4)))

